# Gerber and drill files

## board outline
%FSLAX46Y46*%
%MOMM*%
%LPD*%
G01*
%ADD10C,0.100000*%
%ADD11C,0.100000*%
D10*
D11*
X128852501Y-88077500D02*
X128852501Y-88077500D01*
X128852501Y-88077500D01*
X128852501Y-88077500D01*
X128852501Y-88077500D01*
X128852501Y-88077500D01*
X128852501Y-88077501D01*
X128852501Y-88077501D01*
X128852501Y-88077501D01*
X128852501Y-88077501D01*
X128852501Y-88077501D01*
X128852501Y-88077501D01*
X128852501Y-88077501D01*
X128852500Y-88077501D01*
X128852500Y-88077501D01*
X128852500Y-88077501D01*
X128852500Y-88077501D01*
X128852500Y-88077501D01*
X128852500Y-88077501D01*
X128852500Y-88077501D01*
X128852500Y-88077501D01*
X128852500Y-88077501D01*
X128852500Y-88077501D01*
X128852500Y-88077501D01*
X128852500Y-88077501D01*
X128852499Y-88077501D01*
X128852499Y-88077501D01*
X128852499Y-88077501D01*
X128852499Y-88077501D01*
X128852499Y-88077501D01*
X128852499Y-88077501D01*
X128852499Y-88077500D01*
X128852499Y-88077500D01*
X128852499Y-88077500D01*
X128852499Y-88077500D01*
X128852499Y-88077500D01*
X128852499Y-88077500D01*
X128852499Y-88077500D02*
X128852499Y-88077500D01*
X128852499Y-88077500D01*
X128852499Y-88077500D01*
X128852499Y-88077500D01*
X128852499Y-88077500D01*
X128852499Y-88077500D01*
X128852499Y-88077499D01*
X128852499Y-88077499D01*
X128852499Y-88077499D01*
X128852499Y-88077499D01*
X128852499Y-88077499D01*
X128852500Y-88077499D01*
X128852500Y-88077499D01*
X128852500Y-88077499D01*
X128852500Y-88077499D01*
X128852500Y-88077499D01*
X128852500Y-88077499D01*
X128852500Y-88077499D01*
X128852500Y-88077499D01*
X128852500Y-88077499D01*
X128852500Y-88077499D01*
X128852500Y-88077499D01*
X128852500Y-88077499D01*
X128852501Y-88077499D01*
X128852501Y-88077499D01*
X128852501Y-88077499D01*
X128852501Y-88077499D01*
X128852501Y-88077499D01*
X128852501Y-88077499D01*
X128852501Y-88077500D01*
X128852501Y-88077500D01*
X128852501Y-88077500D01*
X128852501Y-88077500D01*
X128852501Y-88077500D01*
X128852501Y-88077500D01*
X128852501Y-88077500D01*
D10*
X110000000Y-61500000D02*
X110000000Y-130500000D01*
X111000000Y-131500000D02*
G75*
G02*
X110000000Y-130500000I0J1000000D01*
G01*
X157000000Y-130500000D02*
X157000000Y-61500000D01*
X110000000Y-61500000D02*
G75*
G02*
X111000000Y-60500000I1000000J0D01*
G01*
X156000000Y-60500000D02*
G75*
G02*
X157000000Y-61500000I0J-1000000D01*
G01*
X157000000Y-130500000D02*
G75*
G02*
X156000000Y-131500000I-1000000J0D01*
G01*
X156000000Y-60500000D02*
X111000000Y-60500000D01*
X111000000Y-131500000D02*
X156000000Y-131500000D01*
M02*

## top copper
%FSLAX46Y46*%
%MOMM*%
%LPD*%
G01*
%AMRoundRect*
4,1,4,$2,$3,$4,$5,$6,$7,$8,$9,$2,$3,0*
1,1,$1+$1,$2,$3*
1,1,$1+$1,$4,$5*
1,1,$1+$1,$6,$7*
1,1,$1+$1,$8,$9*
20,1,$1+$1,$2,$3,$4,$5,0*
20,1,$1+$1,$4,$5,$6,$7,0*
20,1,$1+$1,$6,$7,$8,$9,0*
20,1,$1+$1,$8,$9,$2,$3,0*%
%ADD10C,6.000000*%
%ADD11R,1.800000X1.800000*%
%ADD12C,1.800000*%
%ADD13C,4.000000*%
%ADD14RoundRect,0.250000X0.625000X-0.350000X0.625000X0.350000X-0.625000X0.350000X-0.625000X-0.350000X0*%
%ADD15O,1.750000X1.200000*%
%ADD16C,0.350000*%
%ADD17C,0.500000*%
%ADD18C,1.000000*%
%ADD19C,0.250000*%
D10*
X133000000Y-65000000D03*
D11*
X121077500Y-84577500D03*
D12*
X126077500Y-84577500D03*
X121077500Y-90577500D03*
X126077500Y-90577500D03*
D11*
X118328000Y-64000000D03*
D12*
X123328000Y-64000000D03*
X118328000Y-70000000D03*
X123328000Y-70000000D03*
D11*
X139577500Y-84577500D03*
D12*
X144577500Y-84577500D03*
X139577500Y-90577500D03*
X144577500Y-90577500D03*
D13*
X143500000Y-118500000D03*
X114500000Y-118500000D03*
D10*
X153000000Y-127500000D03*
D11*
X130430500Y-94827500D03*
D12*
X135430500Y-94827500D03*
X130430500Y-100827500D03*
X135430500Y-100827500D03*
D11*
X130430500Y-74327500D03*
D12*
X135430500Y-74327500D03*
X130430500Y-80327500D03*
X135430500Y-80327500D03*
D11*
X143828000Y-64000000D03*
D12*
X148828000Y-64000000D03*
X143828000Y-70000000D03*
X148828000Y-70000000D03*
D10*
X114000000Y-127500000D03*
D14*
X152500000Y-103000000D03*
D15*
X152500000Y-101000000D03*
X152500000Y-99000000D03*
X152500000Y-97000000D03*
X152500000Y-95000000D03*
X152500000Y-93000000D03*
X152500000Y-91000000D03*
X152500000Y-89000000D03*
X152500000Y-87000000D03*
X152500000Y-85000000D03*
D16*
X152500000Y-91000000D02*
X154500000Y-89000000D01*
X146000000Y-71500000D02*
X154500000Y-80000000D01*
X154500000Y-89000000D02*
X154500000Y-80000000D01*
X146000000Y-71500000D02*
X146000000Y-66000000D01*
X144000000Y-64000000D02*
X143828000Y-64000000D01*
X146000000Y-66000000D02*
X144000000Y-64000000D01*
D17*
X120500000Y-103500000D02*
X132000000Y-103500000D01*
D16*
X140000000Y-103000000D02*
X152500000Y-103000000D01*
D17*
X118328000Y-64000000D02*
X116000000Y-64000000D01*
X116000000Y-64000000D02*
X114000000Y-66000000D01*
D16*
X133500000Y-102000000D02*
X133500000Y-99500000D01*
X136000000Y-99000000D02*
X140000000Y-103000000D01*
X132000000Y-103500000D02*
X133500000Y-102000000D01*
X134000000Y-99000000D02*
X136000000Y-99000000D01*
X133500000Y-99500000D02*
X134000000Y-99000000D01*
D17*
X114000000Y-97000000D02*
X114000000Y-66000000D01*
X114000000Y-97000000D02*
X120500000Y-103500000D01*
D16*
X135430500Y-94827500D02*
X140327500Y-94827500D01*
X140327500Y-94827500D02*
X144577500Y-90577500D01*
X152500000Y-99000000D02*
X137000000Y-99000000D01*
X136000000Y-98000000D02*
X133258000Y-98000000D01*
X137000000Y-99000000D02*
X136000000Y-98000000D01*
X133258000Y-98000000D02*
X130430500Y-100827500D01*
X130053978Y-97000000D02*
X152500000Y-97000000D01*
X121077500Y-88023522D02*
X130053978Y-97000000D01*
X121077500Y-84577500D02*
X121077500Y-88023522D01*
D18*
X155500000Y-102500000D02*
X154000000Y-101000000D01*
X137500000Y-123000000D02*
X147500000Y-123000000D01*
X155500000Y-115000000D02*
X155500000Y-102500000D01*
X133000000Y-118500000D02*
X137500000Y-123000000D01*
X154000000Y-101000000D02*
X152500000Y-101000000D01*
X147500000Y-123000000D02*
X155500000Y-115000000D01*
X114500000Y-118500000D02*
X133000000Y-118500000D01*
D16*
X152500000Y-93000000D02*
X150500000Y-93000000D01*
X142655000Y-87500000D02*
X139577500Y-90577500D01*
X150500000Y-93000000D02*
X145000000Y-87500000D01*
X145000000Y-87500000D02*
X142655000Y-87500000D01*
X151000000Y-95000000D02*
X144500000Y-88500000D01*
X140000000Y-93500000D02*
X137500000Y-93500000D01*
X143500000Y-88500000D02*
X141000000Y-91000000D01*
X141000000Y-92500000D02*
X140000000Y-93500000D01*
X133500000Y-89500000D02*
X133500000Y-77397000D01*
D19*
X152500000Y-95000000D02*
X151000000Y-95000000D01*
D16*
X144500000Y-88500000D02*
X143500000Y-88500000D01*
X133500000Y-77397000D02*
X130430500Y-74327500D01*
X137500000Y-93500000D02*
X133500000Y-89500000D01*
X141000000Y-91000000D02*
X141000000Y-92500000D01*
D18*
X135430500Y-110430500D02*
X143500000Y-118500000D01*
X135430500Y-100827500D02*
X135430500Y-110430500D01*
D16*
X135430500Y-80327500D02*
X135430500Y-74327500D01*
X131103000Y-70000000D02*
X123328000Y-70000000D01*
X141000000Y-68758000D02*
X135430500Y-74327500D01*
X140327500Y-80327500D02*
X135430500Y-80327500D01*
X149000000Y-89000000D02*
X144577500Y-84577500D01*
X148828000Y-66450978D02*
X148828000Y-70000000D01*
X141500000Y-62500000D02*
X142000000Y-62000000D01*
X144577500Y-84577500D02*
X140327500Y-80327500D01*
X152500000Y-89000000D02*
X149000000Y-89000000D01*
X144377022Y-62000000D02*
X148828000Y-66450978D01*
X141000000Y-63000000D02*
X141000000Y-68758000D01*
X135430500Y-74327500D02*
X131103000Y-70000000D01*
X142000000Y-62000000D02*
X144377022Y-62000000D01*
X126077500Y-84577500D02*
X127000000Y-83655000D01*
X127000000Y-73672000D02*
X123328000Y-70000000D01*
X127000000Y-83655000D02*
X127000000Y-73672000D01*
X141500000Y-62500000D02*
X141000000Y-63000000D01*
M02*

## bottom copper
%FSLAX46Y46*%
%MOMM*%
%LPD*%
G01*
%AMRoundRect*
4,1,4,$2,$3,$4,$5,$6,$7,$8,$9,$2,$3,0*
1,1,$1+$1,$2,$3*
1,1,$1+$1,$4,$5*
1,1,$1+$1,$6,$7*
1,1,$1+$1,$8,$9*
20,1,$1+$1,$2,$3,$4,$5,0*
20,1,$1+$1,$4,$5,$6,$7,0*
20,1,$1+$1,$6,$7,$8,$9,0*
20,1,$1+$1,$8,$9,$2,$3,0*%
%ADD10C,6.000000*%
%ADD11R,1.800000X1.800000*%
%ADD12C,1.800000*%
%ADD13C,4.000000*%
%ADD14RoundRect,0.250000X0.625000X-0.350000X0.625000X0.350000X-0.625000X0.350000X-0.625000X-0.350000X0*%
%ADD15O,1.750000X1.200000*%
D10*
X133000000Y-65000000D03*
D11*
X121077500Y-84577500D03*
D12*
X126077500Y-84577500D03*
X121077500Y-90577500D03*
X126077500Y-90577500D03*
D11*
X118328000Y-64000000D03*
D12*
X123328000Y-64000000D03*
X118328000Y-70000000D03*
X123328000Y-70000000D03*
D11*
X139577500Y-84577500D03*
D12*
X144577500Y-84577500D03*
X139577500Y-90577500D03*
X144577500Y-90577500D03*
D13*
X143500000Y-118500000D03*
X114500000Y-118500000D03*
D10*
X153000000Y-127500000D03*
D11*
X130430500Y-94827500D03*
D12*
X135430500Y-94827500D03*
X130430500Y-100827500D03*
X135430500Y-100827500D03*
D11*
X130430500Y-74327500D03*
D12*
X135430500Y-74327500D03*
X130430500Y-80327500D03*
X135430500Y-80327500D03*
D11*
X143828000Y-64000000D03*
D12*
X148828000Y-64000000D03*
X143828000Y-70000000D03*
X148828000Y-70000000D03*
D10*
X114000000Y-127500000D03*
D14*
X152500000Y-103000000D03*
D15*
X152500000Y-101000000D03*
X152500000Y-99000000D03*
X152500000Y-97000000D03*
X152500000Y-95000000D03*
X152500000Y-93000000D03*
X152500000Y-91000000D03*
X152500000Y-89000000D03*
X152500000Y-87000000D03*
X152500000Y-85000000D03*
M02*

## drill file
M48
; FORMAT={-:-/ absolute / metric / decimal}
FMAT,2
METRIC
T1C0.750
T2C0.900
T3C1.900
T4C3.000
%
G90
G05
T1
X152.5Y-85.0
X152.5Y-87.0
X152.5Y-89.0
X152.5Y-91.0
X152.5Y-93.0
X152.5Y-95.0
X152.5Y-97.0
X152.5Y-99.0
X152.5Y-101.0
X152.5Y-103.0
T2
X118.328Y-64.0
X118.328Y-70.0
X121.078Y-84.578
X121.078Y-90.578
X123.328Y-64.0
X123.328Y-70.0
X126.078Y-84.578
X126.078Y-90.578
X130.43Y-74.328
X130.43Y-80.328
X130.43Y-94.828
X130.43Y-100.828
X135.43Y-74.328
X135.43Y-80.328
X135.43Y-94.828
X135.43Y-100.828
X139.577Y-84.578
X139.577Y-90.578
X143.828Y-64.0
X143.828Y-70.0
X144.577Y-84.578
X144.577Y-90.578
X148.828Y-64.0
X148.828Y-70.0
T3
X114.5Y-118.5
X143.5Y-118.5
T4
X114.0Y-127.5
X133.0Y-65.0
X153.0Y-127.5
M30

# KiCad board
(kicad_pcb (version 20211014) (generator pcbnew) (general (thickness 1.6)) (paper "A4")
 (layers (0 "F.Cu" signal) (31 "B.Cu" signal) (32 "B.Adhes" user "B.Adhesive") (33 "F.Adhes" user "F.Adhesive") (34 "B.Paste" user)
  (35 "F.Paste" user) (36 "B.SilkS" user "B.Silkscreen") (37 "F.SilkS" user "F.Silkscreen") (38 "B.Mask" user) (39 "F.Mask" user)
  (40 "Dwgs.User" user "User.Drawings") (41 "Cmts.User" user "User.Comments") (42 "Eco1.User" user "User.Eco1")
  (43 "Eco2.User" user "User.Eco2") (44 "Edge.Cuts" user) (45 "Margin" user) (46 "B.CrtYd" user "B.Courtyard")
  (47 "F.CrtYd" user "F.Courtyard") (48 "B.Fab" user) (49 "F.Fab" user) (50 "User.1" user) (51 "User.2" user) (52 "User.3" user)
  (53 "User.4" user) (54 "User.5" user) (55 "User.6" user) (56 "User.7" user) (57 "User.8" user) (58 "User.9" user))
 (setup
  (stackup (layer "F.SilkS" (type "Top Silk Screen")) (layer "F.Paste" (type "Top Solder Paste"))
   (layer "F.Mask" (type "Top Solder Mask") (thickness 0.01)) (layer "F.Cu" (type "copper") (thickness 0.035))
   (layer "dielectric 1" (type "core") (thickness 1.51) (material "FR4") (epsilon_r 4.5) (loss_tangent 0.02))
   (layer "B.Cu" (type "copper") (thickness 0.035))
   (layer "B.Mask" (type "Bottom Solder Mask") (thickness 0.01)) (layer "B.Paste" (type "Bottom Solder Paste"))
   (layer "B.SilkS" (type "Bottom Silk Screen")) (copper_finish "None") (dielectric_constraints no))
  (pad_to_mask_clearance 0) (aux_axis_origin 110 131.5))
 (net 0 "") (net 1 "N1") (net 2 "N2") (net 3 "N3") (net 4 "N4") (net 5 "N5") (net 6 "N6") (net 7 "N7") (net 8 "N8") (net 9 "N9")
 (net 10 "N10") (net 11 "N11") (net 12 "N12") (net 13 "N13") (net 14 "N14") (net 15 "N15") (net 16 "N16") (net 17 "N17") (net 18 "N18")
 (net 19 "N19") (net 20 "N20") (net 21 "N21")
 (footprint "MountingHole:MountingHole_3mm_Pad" (layer "F.Cu") (at 133 65)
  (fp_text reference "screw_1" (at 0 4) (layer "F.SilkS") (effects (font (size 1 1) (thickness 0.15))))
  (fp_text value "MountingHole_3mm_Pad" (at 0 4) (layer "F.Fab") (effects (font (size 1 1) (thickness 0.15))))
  (pad "1" thru_hole circle (at 0 0) (size 6 6) (drill 3) (layers *.Cu *.Mask)))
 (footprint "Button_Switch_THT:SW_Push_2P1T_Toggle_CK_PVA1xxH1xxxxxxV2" (layer "F.Cu") (at 121.0775 84.5775)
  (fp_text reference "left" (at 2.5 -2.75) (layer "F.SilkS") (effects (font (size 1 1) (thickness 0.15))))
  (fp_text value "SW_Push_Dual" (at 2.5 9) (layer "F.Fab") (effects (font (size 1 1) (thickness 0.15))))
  (pad "1" thru_hole rect (at 0 0) (size 1.8 1.8) (drill 0.9) (layers *.Cu *.Mask) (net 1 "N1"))
  (pad "2" thru_hole circle (at 5 0) (size 1.8 1.8) (drill 0.9) (layers *.Cu *.Mask) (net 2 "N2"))
  (pad "3" thru_hole circle (at 0 6) (size 1.8 1.8) (drill 0.9) (layers *.Cu *.Mask) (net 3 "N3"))
  (pad "4" thru_hole circle (at 5 6) (size 1.8 1.8) (drill 0.9) (layers *.Cu *.Mask) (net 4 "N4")))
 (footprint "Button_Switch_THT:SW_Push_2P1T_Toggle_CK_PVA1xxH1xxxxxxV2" (layer "F.Cu") (at 118.328 64)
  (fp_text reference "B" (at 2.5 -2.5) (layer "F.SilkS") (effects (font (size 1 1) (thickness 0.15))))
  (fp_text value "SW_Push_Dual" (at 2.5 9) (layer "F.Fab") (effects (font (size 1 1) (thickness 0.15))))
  (pad "1" thru_hole rect (at 0 0) (size 1.8 1.8) (drill 0.9) (layers *.Cu *.Mask) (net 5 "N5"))
  (pad "2" thru_hole circle (at 5 0) (size 1.8 1.8) (drill 0.9) (layers *.Cu *.Mask) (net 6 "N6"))
  (pad "3" thru_hole circle (at 0 6) (size 1.8 1.8) (drill 0.9) (layers *.Cu *.Mask) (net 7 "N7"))
  (pad "4" thru_hole circle (at 5 6) (size 1.8 1.8) (drill 0.9) (layers *.Cu *.Mask) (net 2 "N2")))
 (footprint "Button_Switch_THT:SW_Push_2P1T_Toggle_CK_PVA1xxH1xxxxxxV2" (layer "F.Cu") (at 139.5775 84.5775)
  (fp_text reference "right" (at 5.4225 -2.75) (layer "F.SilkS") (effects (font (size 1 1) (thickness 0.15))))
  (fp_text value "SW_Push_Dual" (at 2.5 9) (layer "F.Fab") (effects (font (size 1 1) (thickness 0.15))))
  (pad "1" thru_hole rect (at 0 0) (size 1.8 1.8) (drill 0.9) (layers *.Cu *.Mask) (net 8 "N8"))
  (pad "2" thru_hole circle (at 5 0) (size 1.8 1.8) (drill 0.9) (layers *.Cu *.Mask) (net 2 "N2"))
  (pad "3" thru_hole circle (at 0 6) (size 1.8 1.8) (drill 0.9) (layers *.Cu *.Mask) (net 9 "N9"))
  (pad "4" thru_hole circle (at 5 6) (size 1.8 1.8) (drill 0.9) (layers *.Cu *.Mask) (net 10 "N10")))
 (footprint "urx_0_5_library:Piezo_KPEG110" (layer "F.Cu") (at 129 118.5)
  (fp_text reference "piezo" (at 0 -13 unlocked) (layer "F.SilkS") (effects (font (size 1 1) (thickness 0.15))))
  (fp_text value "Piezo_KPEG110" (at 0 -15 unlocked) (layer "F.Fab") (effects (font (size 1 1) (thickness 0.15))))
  (pad "1" thru_hole circle (at 14.5 0) (size 4 4) (drill 1.9) (layers *.Cu *.Mask) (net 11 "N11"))
  (pad "2" thru_hole circle (at -14.5 0) (size 4 4) (drill 1.9) (layers *.Cu *.Mask) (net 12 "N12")))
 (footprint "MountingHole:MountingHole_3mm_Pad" (layer "F.Cu") (at 153 127.5)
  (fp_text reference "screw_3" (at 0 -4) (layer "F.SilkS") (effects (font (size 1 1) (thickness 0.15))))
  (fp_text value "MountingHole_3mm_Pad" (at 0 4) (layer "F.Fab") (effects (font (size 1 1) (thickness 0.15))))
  (pad "1" thru_hole circle (at 0 0) (size 6 6) (drill 3) (layers *.Cu *.Mask)))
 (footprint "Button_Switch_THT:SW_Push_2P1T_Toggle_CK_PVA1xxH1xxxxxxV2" (layer "F.Cu") (at 130.4305 94.8275)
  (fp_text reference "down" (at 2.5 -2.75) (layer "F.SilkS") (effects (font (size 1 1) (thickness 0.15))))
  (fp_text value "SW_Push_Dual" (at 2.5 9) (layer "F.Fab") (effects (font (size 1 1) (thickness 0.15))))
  (pad "1" thru_hole rect (at 0 0) (size 1.8 1.8) (drill 0.9) (layers *.Cu *.Mask) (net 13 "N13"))
  (pad "2" thru_hole circle (at 5 0) (size 1.8 1.8) (drill 0.9) (layers *.Cu *.Mask) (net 10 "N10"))
  (pad "3" thru_hole circle (at 0 6) (size 1.8 1.8) (drill 0.9) (layers *.Cu *.Mask) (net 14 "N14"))
  (pad "4" thru_hole circle (at 5 6) (size 1.8 1.8) (drill 0.9) (layers *.Cu *.Mask) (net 11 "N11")))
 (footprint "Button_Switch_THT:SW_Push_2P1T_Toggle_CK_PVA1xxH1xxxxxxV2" (layer "F.Cu") (at 130.4305 74.3275)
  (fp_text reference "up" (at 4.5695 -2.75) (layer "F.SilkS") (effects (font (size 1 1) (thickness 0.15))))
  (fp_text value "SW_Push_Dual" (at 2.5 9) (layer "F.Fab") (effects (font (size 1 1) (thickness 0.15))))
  (pad "1" thru_hole rect (at 0 0) (size 1.8 1.8) (drill 0.9) (layers *.Cu *.Mask) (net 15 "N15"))
  (pad "2" thru_hole circle (at 5 0) (size 1.8 1.8) (drill 0.9) (layers *.Cu *.Mask) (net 2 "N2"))
  (pad "3" thru_hole circle (at 0 6) (size 1.8 1.8) (drill 0.9) (layers *.Cu *.Mask) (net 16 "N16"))
  (pad "4" thru_hole circle (at 5 6) (size 1.8 1.8) (drill 0.9) (layers *.Cu *.Mask) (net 2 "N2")))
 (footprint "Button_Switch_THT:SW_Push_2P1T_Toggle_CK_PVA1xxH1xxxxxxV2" (layer "F.Cu") (at 143.828 64)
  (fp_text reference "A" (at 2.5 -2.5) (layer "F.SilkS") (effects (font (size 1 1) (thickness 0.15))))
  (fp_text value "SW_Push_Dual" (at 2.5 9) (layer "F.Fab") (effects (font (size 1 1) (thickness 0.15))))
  (pad "1" thru_hole rect (at 0 0) (size 1.8 1.8) (drill 0.9) (layers *.Cu *.Mask) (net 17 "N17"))
  (pad "2" thru_hole circle (at 5 0) (size 1.8 1.8) (drill 0.9) (layers *.Cu *.Mask) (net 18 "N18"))
  (pad "3" thru_hole circle (at 0 6) (size 1.8 1.8) (drill 0.9) (layers *.Cu *.Mask) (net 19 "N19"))
  (pad "4" thru_hole circle (at 5 6) (size 1.8 1.8) (drill 0.9) (layers *.Cu *.Mask) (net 2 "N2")))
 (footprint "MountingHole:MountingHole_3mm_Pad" (layer "F.Cu") (at 114 127.5)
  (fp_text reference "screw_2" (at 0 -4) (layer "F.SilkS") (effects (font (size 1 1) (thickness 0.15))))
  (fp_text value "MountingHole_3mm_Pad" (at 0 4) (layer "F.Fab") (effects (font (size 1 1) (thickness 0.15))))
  (pad "1" thru_hole circle (at 0 0) (size 6 6) (drill 3) (layers *.Cu *.Mask)))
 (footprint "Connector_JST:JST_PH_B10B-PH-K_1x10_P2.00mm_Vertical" (layer "F.Cu") (at 152.5 103 90)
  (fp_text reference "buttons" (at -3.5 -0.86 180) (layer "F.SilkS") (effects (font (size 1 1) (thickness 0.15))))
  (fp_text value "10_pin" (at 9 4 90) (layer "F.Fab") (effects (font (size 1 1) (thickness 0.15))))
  (pad "1" thru_hole roundrect (at 0 0 90) (size 1.2 1.75) (drill 0.75) (layers *.Cu *.Mask) (roundrect_rratio 0.2083333333) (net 5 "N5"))
  (pad "2" thru_hole oval (at 2 0 90) (size 1.2 1.75) (drill 0.75) (layers *.Cu *.Mask) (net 12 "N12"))
  (pad "3" thru_hole oval (at 4 0 90) (size 1.2 1.75) (drill 0.75) (layers *.Cu *.Mask) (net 14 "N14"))
  (pad "4" thru_hole oval (at 6 0 90) (size 1.2 1.75) (drill 0.75) (layers *.Cu *.Mask) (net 1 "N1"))
  (pad "5" thru_hole oval (at 8 0 90) (size 1.2 1.75) (drill 0.75) (layers *.Cu *.Mask) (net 15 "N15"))
  (pad "6" thru_hole oval (at 10 0 90) (size 1.2 1.75) (drill 0.75) (layers *.Cu *.Mask) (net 9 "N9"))
  (pad "7" thru_hole oval (at 12 0 90) (size 1.2 1.75) (drill 0.75) (layers *.Cu *.Mask) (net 17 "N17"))
  (pad "8" thru_hole oval (at 14 0 90) (size 1.2 1.75) (drill 0.75) (layers *.Cu *.Mask) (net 2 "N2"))
  (pad "9" thru_hole oval (at 16 0 90) (size 1.2 1.75) (drill 0.75) (layers *.Cu *.Mask) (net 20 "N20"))
  (pad "10" thru_hole oval (at 18 0 90) (size 1.2 1.75) (drill 0.75) (layers *.Cu *.Mask) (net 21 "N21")))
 (gr_circle (center 128.8525 88.0775) (end 128.8525 88.0775) (layer "Edge.Cuts") (width 0.1) (fill none))
 (gr_line (start 110 61.5) (end 110 130.5) (layer "Edge.Cuts") (width 0.1))
 (gr_arc (start 111 131.5) (mid 110.292893 131.207107) (end 110 130.5) (layer "Edge.Cuts") (width 0.1))
 (gr_line (start 157 130.5) (end 157 61.5) (layer "Edge.Cuts") (width 0.1))
 (gr_arc (start 110 61.5) (mid 110.292893 60.792893) (end 111 60.5) (layer "Edge.Cuts") (width 0.1))
 (gr_arc (start 156 60.5) (mid 156.707107 60.792893) (end 157 61.5) (layer "Edge.Cuts") (width 0.1))
 (gr_arc (start 157 130.5) (mid 156.707107 131.207107) (end 156 131.5) (layer "Edge.Cuts") (width 0.1))
 (gr_line (start 156 60.5) (end 111 60.5) (layer "Edge.Cuts") (width 0.1))
 (gr_line (start 111 131.5) (end 156 131.5) (layer "Edge.Cuts") (width 0.1))
 (segment (start 152.5 91) (end 154.5 89) (width 0.35) (layer "F.Cu") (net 17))
 (segment (start 146 71.5) (end 154.5 80) (width 0.35) (layer "F.Cu") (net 17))
 (segment (start 154.5 89) (end 154.5 80) (width 0.35) (layer "F.Cu") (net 17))
 (segment (start 146 71.5) (end 146 66) (width 0.35) (layer "F.Cu") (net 17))
 (segment (start 144 64) (end 143.828 64) (width 0.35) (layer "F.Cu") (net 17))
 (segment (start 146 66) (end 144 64) (width 0.35) (layer "F.Cu") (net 17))
 (segment (start 120.5 103.5) (end 132 103.5) (width 0.5) (layer "F.Cu") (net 5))
 (segment (start 140 103) (end 152.5 103) (width 0.35) (layer "F.Cu") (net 5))
 (segment (start 118.328 64) (end 116 64) (width 0.5) (layer "F.Cu") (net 5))
 (segment (start 116 64) (end 114 66) (width 0.5) (layer "F.Cu") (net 5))
 (segment (start 133.5 102) (end 133.5 99.5) (width 0.35) (layer "F.Cu") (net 5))
 (segment (start 136 99) (end 140 103) (width 0.35) (layer "F.Cu") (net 5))
 (segment (start 132 103.5) (end 133.5 102) (width 0.35) (layer "F.Cu") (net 5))
 (segment (start 134 99) (end 136 99) (width 0.35) (layer "F.Cu") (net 5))
 (segment (start 133.5 99.5) (end 134 99) (width 0.35) (layer "F.Cu") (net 5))
 (segment (start 114 97) (end 114 66) (width 0.5) (layer "F.Cu") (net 5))
 (segment (start 114 97) (end 120.5 103.5) (width 0.5) (layer "F.Cu") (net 5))
 (segment (start 135.4305 94.8275) (end 140.3275 94.8275) (width 0.35) (layer "F.Cu") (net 10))
 (segment (start 140.3275 94.8275) (end 144.5775 90.5775) (width 0.35) (layer "F.Cu") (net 10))
 (segment (start 152.5 99) (end 137 99) (width 0.35) (layer "F.Cu") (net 14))
 (segment (start 136 98) (end 133.258 98) (width 0.35) (layer "F.Cu") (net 14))
 (segment (start 137 99) (end 136 98) (width 0.35) (layer "F.Cu") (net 14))
 (segment (start 133.258 98) (end 130.4305 100.8275) (width 0.35) (layer "F.Cu") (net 14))
 (segment (start 130.053978 97) (end 152.5 97) (width 0.35) (layer "F.Cu") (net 1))
 (segment (start 121.0775 88.023522) (end 130.053978 97) (width 0.35) (layer "F.Cu") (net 1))
 (segment (start 121.0775 84.5775) (end 121.0775 88.023522) (width 0.35) (layer "F.Cu") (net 1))
 (segment (start 155.5 102.5) (end 154 101) (width 1) (layer "F.Cu") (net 12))
 (segment (start 137.5 123) (end 147.5 123) (width 1) (layer "F.Cu") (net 12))
 (segment (start 155.5 115) (end 155.5 102.5) (width 1) (layer "F.Cu") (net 12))
 (segment (start 133 118.5) (end 137.5 123) (width 1) (layer "F.Cu") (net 12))
 (segment (start 154 101) (end 152.5 101) (width 1) (layer "F.Cu") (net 12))
 (segment (start 147.5 123) (end 155.5 115) (width 1) (layer "F.Cu") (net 12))
 (segment (start 114.5 118.5) (end 133 118.5) (width 1) (layer "F.Cu") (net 12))
 (segment (start 152.5 93) (end 150.5 93) (width 0.35) (layer "F.Cu") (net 9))
 (segment (start 142.655 87.5) (end 139.5775 90.5775) (width 0.35) (layer "F.Cu") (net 9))
 (segment (start 150.5 93) (end 145 87.5) (width 0.35) (layer "F.Cu") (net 9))
 (segment (start 145 87.5) (end 142.655 87.5) (width 0.35) (layer "F.Cu") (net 9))
 (segment (start 151 95) (end 144.5 88.5) (width 0.35) (layer "F.Cu") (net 15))
 (segment (start 140 93.5) (end 137.5 93.5) (width 0.35) (layer "F.Cu") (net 15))
 (segment (start 143.5 88.5) (end 141 91) (width 0.35) (layer "F.Cu") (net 15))
 (segment (start 141 92.5) (end 140 93.5) (width 0.35) (layer "F.Cu") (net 15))
 (segment (start 133.5 89.5) (end 133.5 77.397) (width 0.35) (layer "F.Cu") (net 15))
 (segment (start 152.5 95) (end 151 95) (width 0.25) (layer "F.Cu") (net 15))
 (segment (start 144.5 88.5) (end 143.5 88.5) (width 0.35) (layer "F.Cu") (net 15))
 (segment (start 133.5 77.397) (end 130.4305 74.3275) (width 0.35) (layer "F.Cu") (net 15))
 (segment (start 137.5 93.5) (end 133.5 89.5) (width 0.35) (layer "F.Cu") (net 15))
 (segment (start 141 91) (end 141 92.5) (width 0.35) (layer "F.Cu") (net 15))
 (segment (start 135.4305 110.4305) (end 143.5 118.5) (width 1) (layer "F.Cu") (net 11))
 (segment (start 135.4305 100.8275) (end 135.4305 110.4305) (width 1) (layer "F.Cu") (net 11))
 (segment (start 135.4305 80.3275) (end 135.4305 74.3275) (width 0.35) (layer "F.Cu") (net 2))
 (segment (start 131.103 70) (end 123.328 70) (width 0.35) (layer "F.Cu") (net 2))
 (segment (start 141 68.758) (end 135.4305 74.3275) (width 0.35) (layer "F.Cu") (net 2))
 (segment (start 140.3275 80.3275) (end 135.4305 80.3275) (width 0.35) (layer "F.Cu") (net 2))
 (segment (start 149 89) (end 144.5775 84.5775) (width 0.35) (layer "F.Cu") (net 2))
 (segment (start 148.828 66.450978) (end 148.828 70) (width 0.35) (layer "F.Cu") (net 2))
 (segment (start 141.5 62.5) (end 142 62) (width 0.35) (layer "F.Cu") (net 2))
 (segment (start 144.5775 84.5775) (end 140.3275 80.3275) (width 0.35) (layer "F.Cu") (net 2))
 (segment (start 152.5 89) (end 149 89) (width 0.35) (layer "F.Cu") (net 2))
 (segment (start 144.377022 62) (end 148.828 66.450978) (width 0.35) (layer "F.Cu") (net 2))
 (segment (start 141 63) (end 141 68.758) (width 0.35) (layer "F.Cu") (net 2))
 (segment (start 135.4305 74.3275) (end 131.103 70) (width 0.35) (layer "F.Cu") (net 2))
 (segment (start 142 62) (end 144.377022 62) (width 0.35) (layer "F.Cu") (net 2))
 (segment (start 126.0775 84.5775) (end 127 83.655) (width 0.35) (layer "F.Cu") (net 2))
 (segment (start 127 73.672) (end 123.328 70) (width 0.35) (layer "F.Cu") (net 2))
 (segment (start 127 83.655) (end 127 73.672) (width 0.35) (layer "F.Cu") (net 2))
 (segment (start 141.5 62.5) (end 141 63) (width 0.35) (layer "F.Cu") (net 2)))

